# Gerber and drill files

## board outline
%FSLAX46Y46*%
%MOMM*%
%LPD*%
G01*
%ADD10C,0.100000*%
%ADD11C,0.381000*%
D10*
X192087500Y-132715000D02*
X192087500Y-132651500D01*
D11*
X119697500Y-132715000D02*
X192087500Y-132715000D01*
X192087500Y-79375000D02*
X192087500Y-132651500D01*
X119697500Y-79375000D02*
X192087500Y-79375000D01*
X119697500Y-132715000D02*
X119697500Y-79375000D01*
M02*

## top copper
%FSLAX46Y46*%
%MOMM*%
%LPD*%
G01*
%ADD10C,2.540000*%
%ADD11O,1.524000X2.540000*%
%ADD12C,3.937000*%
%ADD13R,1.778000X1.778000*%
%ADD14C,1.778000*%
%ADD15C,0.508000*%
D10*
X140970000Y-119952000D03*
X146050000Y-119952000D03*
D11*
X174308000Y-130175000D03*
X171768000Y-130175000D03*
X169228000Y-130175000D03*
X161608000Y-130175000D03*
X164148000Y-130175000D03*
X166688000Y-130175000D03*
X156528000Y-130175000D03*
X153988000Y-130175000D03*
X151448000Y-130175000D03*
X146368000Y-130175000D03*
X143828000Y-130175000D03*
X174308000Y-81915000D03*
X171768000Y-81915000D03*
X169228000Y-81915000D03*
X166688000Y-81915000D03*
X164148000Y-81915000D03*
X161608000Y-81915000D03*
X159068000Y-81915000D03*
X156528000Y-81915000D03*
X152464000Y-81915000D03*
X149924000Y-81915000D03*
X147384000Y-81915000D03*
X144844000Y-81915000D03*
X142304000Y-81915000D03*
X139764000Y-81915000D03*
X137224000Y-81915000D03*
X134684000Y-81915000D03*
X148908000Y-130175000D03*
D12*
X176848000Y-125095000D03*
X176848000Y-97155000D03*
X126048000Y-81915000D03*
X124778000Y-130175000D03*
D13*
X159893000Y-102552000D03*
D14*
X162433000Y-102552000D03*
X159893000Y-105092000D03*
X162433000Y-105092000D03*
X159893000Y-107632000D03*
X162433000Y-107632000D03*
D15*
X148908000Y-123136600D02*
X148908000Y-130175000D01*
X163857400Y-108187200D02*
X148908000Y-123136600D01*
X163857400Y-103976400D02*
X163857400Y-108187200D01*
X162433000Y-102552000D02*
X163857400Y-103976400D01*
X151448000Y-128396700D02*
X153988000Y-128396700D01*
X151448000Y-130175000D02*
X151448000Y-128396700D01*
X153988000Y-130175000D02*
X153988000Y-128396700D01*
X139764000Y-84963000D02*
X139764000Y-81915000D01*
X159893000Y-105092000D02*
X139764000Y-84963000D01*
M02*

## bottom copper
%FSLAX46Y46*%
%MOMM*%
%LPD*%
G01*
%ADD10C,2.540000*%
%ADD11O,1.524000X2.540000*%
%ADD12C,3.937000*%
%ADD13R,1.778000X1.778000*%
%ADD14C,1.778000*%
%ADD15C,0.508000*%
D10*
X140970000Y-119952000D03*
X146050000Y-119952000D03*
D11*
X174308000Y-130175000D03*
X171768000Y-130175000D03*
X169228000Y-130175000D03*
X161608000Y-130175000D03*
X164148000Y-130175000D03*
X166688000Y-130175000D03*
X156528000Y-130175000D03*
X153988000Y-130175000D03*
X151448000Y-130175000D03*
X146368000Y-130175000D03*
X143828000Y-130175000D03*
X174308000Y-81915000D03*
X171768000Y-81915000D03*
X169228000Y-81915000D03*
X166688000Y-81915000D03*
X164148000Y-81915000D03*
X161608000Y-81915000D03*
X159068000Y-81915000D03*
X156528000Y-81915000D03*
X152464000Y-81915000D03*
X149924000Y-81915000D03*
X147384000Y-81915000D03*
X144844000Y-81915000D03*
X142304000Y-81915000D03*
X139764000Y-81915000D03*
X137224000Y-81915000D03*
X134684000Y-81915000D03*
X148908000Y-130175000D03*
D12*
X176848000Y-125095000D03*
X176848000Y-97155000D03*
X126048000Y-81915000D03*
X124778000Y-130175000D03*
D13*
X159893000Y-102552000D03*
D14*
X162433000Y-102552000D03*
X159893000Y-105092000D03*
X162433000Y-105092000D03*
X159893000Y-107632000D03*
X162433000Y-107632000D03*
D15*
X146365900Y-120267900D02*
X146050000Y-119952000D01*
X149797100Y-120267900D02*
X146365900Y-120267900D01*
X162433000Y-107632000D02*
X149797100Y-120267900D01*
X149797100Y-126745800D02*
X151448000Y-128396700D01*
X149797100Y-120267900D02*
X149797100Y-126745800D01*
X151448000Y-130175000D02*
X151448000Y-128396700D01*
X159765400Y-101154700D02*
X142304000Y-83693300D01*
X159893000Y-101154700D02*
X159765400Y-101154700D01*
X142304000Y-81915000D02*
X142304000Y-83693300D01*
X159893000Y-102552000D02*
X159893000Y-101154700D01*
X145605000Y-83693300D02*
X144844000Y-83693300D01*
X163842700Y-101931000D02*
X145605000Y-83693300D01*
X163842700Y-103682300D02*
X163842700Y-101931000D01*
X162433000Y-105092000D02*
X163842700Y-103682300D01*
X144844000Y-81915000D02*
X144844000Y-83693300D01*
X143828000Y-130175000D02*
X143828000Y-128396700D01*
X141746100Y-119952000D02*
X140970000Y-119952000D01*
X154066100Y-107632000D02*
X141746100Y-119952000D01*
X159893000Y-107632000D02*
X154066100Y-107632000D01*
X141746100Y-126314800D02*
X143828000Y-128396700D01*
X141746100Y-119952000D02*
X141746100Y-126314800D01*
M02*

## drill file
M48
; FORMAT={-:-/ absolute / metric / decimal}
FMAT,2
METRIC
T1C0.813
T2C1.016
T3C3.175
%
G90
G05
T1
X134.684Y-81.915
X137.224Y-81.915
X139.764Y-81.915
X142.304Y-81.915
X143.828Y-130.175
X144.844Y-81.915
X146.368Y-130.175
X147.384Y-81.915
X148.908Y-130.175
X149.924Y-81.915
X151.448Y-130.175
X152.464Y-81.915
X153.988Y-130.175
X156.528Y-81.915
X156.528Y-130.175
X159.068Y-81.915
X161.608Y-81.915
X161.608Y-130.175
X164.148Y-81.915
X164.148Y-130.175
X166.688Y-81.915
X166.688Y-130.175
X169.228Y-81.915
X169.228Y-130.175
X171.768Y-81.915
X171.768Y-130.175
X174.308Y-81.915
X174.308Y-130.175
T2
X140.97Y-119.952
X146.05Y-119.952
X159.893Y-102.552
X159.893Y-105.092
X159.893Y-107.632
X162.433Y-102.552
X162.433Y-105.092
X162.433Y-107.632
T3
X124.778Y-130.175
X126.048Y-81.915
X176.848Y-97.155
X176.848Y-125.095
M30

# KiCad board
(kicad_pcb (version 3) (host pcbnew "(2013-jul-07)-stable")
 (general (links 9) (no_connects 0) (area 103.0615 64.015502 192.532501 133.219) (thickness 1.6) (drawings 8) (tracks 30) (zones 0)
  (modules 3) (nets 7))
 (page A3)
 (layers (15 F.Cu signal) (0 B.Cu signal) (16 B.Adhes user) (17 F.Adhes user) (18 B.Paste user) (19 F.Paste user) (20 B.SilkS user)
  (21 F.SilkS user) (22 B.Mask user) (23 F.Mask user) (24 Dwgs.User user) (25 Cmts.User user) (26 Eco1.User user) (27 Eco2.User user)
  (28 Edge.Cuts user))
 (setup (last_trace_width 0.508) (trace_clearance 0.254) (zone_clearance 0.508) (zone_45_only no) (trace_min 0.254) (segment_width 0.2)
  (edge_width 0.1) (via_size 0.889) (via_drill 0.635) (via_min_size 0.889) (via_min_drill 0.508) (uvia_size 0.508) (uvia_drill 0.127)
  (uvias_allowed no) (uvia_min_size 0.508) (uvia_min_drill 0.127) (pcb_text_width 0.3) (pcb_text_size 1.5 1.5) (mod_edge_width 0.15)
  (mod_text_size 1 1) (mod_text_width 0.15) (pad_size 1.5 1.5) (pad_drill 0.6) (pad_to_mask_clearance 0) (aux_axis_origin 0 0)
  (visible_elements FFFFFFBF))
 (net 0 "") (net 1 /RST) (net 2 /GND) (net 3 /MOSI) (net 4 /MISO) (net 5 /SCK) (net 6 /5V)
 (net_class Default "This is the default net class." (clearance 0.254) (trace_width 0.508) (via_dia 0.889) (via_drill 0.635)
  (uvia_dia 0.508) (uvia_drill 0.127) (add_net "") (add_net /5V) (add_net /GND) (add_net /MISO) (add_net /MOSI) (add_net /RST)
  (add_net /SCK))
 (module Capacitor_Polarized (layer F.Cu) (at 143.51 119.952)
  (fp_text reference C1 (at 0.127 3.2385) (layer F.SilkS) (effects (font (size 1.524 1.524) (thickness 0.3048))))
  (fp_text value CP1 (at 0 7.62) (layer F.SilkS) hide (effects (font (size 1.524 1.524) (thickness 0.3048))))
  (pad 1 thru_hole circle (at -2.54 0) (size 2.54 2.54) (drill 1.016) (layers *.Cu *.SilkS *.Mask) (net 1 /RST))
  (pad 2 thru_hole circle (at 2.54 0) (size 2.54 2.54) (drill 1.016) (layers *.Cu *.SilkS *.Mask) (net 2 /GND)))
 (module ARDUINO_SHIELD (layer F.Cu) (at 119.698 132.715)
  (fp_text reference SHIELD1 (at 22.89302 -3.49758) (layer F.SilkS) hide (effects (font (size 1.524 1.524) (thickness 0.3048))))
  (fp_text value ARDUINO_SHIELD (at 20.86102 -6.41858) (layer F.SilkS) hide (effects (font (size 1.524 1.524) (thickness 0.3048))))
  (pad AD5 thru_hole oval (at 54.61 -2.54 90) (size 2.54 1.524) (drill 0.8128) (layers *.Cu *.Mask F.SilkS))
  (pad AD4 thru_hole oval (at 52.07 -2.54 90) (size 2.54 1.524) (drill 0.8128) (layers *.Cu *.Mask F.SilkS))
  (pad AD3 thru_hole oval (at 49.53 -2.54 90) (size 2.54 1.524) (drill 0.8128) (layers *.Cu *.Mask F.SilkS))
  (pad AD0 thru_hole oval (at 41.91 -2.54 90) (size 2.54 1.524) (drill 0.8128) (layers *.Cu *.Mask F.SilkS))
  (pad AD1 thru_hole oval (at 44.45 -2.54 90) (size 2.54 1.524) (drill 0.8128) (layers *.Cu *.Mask F.SilkS))
  (pad AD2 thru_hole oval (at 46.99 -2.54 90) (size 2.54 1.524) (drill 0.8128) (layers *.Cu *.Mask F.SilkS))
  (pad V_IN thru_hole oval (at 36.83 -2.54 90) (size 2.54 1.524) (drill 0.8128) (layers *.Cu *.Mask F.SilkS))
  (pad GND2 thru_hole oval (at 34.29 -2.54 90) (size 2.54 1.524) (drill 0.8128) (layers *.Cu *.Mask F.SilkS) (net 2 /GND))
  (pad GND1 thru_hole oval (at 31.75 -2.54 90) (size 2.54 1.524) (drill 0.8128) (layers *.Cu *.Mask F.SilkS) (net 2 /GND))
  (pad 3V3 thru_hole oval (at 26.67 -2.54 90) (size 2.54 1.524) (drill 0.8128) (layers *.Cu *.Mask F.SilkS))
  (pad RST thru_hole oval (at 24.13 -2.54 90) (size 2.54 1.524) (drill 0.8128) (layers *.Cu *.Mask F.SilkS) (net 1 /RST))
  (pad 0 thru_hole oval (at 54.61 -50.8 90) (size 2.54 1.524) (drill 0.8128) (layers *.Cu *.Mask F.SilkS))
  (pad 1 thru_hole oval (at 52.07 -50.8 90) (size 2.54 1.524) (drill 0.8128) (layers *.Cu *.Mask F.SilkS))
  (pad 2 thru_hole oval (at 49.53 -50.8 90) (size 2.54 1.524) (drill 0.8128) (layers *.Cu *.Mask F.SilkS))
  (pad 3 thru_hole oval (at 46.99 -50.8 90) (size 2.54 1.524) (drill 0.8128) (layers *.Cu *.Mask F.SilkS))
  (pad 4 thru_hole oval (at 44.45 -50.8 90) (size 2.54 1.524) (drill 0.8128) (layers *.Cu *.Mask F.SilkS))
  (pad 5 thru_hole oval (at 41.91 -50.8 90) (size 2.54 1.524) (drill 0.8128) (layers *.Cu *.Mask F.SilkS))
  (pad 6 thru_hole oval (at 39.37 -50.8 90) (size 2.54 1.524) (drill 0.8128) (layers *.Cu *.Mask F.SilkS))
  (pad 7 thru_hole oval (at 36.83 -50.8 90) (size 2.54 1.524) (drill 0.8128) (layers *.Cu *.Mask F.SilkS))
  (pad 8 thru_hole oval (at 32.766 -50.8 90) (size 2.54 1.524) (drill 0.8128) (layers *.Cu *.Mask F.SilkS))
  (pad 9 thru_hole oval (at 30.226 -50.8 90) (size 2.54 1.524) (drill 0.8128) (layers *.Cu *.Mask F.SilkS))
  (pad 10 thru_hole oval (at 27.686 -50.8 90) (size 2.54 1.524) (drill 0.8128) (layers *.Cu *.Mask F.SilkS))
  (pad 11 thru_hole oval (at 25.146 -50.8 90) (size 2.54 1.524) (drill 0.8128) (layers *.Cu *.Mask F.SilkS) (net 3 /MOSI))
  (pad 12 thru_hole oval (at 22.606 -50.8 90) (size 2.54 1.524) (drill 0.8128) (layers *.Cu *.Mask F.SilkS) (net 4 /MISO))
  (pad 13 thru_hole oval (at 20.066 -50.8 90) (size 2.54 1.524) (drill 0.8128) (layers *.Cu *.Mask F.SilkS) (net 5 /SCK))
  (pad GND3 thru_hole oval (at 17.526 -50.8 90) (size 2.54 1.524) (drill 0.8128) (layers *.Cu *.Mask F.SilkS))
  (pad AREF thru_hole oval (at 14.986 -50.8 90) (size 2.54 1.524) (drill 0.8128) (layers *.Cu *.Mask F.SilkS))
  (pad 5V thru_hole oval (at 29.21 -2.54 90) (size 2.54 1.524) (drill 0.8128) (layers *.Cu *.Mask F.SilkS) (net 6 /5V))
  (pad "" thru_hole circle (at 57.15 -7.62 90) (size 3.937 3.937) (drill 3.175) (layers *.Cu *.Mask F.SilkS))
  (pad "" thru_hole circle (at 57.15 -35.56 90) (size 3.937 3.937) (drill 3.175) (layers *.Cu *.Mask F.SilkS))
  (pad "" thru_hole circle (at 6.35 -50.8 90) (size 3.937 3.937) (drill 3.175) (layers *.Cu *.Mask F.SilkS))
  (pad "" thru_hole circle (at 5.08 -2.54 90) (size 3.937 3.937) (drill 3.175) (layers *.Cu *.Mask F.SilkS)))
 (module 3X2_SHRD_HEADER (layer F.Cu) (at 161.163 105.092 270)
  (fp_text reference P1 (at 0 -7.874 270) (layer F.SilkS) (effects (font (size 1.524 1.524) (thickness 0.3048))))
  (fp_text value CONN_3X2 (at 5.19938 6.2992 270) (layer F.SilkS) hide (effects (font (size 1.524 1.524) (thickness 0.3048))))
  (pad 1 thru_hole rect (at -2.54 1.27 270) (size 1.778 1.778) (drill 1.016) (layers *.Cu *.Mask F.SilkS) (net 4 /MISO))
  (pad 2 thru_hole circle (at -2.54 -1.27 270) (size 1.778 1.778) (drill 1.016) (layers *.Cu *.Mask F.SilkS) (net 6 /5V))
  (pad 3 thru_hole circle (at 0 1.27 270) (size 1.778 1.778) (drill 1.016) (layers *.Cu *.Mask F.SilkS) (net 5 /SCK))
  (pad 4 thru_hole circle (at 0 -1.27 270) (size 1.778 1.778) (drill 1.016) (layers *.Cu *.Mask F.SilkS) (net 3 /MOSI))
  (pad 5 thru_hole circle (at 2.54 1.27 270) (size 1.778 1.778) (drill 1.016) (layers *.Cu *.Mask F.SilkS) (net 1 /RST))
  (pad 6 thru_hole circle (at 2.54 -1.27 270) (size 1.778 1.778) (drill 1.016) (layers *.Cu *.Mask F.SilkS) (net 2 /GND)))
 (gr_line (start 192.0875 132.715) (end 192.0875 132.6515) (angle 90) (layer Edge.Cuts) (width 0.1))
 (gr_line (start 119.6975 132.715) (end 192.0875 132.715) (angle 90) (layer Edge.Cuts) (width 0.381))
 (gr_line (start 192.0875 79.375) (end 192.0875 132.6515) (angle 90) (layer Edge.Cuts) (width 0.381))
 (gr_line (start 119.6975 79.375) (end 192.0875 79.375) (angle 90) (layer Edge.Cuts) (width 0.381))
 (gr_line (start 119.6975 132.715) (end 119.6975 79.375) (angle 90) (layer Edge.Cuts) (width 0.381))
 (segment (start 148.908 123.1366) (end 148.908 130.175) (width 0.508) (layer F.Cu) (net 6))
 (segment (start 163.8574 108.1872) (end 148.908 123.1366) (width 0.508) (layer F.Cu) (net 6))
 (segment (start 163.8574 103.9764) (end 163.8574 108.1872) (width 0.508) (layer F.Cu) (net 6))
 (segment (start 162.433 102.552) (end 163.8574 103.9764) (width 0.508) (layer F.Cu) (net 6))
 (segment (start 151.448 128.3967) (end 153.988 128.3967) (width 0.508) (layer F.Cu) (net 2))
 (segment (start 151.448 130.175) (end 151.448 128.3967) (width 0.508) (layer F.Cu) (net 2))
 (segment (start 153.988 130.175) (end 153.988 128.3967) (width 0.508) (layer F.Cu) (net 2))
 (segment (start 146.3659 120.2679) (end 146.05 119.952) (width 0.508) (layer B.Cu) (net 2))
 (segment (start 149.7971 120.2679) (end 146.3659 120.2679) (width 0.508) (layer B.Cu) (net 2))
 (segment (start 162.433 107.632) (end 149.7971 120.2679) (width 0.508) (layer B.Cu) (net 2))
 (segment (start 149.7971 126.7458) (end 151.448 128.3967) (width 0.508) (layer B.Cu) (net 2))
 (segment (start 149.7971 120.2679) (end 149.7971 126.7458) (width 0.508) (layer B.Cu) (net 2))
 (segment (start 151.448 130.175) (end 151.448 128.3967) (width 0.508) (layer B.Cu) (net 2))
 (segment (start 159.7654 101.1547) (end 142.304 83.6933) (width 0.508) (layer B.Cu) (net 4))
 (segment (start 159.893 101.1547) (end 159.7654 101.1547) (width 0.508) (layer B.Cu) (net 4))
 (segment (start 142.304 81.915) (end 142.304 83.6933) (width 0.508) (layer B.Cu) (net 4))
 (segment (start 159.893 102.552) (end 159.893 101.1547) (width 0.508) (layer B.Cu) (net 4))
 (segment (start 145.605 83.6933) (end 144.844 83.6933) (width 0.508) (layer B.Cu) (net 3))
 (segment (start 163.8427 101.931) (end 145.605 83.6933) (width 0.508) (layer B.Cu) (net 3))
 (segment (start 163.8427 103.6823) (end 163.8427 101.931) (width 0.508) (layer B.Cu) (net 3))
 (segment (start 162.433 105.092) (end 163.8427 103.6823) (width 0.508) (layer B.Cu) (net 3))
 (segment (start 144.844 81.915) (end 144.844 83.6933) (width 0.508) (layer B.Cu) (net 3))
 (segment (start 143.828 130.175) (end 143.828 128.3967) (width 0.508) (layer B.Cu) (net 1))
 (segment (start 141.7461 119.952) (end 140.97 119.952) (width 0.508) (layer B.Cu) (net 1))
 (segment (start 154.0661 107.632) (end 141.7461 119.952) (width 0.508) (layer B.Cu) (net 1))
 (segment (start 159.893 107.632) (end 154.0661 107.632) (width 0.508) (layer B.Cu) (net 1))
 (segment (start 141.7461 126.3148) (end 143.828 128.3967) (width 0.508) (layer B.Cu) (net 1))
 (segment (start 141.7461 119.952) (end 141.7461 126.3148) (width 0.508) (layer B.Cu) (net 1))
 (segment (start 139.764 84.963) (end 139.764 81.915) (width 0.508) (layer F.Cu) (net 5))
 (segment (start 159.893 105.092) (end 139.764 84.963) (width 0.508) (layer F.Cu) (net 5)))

